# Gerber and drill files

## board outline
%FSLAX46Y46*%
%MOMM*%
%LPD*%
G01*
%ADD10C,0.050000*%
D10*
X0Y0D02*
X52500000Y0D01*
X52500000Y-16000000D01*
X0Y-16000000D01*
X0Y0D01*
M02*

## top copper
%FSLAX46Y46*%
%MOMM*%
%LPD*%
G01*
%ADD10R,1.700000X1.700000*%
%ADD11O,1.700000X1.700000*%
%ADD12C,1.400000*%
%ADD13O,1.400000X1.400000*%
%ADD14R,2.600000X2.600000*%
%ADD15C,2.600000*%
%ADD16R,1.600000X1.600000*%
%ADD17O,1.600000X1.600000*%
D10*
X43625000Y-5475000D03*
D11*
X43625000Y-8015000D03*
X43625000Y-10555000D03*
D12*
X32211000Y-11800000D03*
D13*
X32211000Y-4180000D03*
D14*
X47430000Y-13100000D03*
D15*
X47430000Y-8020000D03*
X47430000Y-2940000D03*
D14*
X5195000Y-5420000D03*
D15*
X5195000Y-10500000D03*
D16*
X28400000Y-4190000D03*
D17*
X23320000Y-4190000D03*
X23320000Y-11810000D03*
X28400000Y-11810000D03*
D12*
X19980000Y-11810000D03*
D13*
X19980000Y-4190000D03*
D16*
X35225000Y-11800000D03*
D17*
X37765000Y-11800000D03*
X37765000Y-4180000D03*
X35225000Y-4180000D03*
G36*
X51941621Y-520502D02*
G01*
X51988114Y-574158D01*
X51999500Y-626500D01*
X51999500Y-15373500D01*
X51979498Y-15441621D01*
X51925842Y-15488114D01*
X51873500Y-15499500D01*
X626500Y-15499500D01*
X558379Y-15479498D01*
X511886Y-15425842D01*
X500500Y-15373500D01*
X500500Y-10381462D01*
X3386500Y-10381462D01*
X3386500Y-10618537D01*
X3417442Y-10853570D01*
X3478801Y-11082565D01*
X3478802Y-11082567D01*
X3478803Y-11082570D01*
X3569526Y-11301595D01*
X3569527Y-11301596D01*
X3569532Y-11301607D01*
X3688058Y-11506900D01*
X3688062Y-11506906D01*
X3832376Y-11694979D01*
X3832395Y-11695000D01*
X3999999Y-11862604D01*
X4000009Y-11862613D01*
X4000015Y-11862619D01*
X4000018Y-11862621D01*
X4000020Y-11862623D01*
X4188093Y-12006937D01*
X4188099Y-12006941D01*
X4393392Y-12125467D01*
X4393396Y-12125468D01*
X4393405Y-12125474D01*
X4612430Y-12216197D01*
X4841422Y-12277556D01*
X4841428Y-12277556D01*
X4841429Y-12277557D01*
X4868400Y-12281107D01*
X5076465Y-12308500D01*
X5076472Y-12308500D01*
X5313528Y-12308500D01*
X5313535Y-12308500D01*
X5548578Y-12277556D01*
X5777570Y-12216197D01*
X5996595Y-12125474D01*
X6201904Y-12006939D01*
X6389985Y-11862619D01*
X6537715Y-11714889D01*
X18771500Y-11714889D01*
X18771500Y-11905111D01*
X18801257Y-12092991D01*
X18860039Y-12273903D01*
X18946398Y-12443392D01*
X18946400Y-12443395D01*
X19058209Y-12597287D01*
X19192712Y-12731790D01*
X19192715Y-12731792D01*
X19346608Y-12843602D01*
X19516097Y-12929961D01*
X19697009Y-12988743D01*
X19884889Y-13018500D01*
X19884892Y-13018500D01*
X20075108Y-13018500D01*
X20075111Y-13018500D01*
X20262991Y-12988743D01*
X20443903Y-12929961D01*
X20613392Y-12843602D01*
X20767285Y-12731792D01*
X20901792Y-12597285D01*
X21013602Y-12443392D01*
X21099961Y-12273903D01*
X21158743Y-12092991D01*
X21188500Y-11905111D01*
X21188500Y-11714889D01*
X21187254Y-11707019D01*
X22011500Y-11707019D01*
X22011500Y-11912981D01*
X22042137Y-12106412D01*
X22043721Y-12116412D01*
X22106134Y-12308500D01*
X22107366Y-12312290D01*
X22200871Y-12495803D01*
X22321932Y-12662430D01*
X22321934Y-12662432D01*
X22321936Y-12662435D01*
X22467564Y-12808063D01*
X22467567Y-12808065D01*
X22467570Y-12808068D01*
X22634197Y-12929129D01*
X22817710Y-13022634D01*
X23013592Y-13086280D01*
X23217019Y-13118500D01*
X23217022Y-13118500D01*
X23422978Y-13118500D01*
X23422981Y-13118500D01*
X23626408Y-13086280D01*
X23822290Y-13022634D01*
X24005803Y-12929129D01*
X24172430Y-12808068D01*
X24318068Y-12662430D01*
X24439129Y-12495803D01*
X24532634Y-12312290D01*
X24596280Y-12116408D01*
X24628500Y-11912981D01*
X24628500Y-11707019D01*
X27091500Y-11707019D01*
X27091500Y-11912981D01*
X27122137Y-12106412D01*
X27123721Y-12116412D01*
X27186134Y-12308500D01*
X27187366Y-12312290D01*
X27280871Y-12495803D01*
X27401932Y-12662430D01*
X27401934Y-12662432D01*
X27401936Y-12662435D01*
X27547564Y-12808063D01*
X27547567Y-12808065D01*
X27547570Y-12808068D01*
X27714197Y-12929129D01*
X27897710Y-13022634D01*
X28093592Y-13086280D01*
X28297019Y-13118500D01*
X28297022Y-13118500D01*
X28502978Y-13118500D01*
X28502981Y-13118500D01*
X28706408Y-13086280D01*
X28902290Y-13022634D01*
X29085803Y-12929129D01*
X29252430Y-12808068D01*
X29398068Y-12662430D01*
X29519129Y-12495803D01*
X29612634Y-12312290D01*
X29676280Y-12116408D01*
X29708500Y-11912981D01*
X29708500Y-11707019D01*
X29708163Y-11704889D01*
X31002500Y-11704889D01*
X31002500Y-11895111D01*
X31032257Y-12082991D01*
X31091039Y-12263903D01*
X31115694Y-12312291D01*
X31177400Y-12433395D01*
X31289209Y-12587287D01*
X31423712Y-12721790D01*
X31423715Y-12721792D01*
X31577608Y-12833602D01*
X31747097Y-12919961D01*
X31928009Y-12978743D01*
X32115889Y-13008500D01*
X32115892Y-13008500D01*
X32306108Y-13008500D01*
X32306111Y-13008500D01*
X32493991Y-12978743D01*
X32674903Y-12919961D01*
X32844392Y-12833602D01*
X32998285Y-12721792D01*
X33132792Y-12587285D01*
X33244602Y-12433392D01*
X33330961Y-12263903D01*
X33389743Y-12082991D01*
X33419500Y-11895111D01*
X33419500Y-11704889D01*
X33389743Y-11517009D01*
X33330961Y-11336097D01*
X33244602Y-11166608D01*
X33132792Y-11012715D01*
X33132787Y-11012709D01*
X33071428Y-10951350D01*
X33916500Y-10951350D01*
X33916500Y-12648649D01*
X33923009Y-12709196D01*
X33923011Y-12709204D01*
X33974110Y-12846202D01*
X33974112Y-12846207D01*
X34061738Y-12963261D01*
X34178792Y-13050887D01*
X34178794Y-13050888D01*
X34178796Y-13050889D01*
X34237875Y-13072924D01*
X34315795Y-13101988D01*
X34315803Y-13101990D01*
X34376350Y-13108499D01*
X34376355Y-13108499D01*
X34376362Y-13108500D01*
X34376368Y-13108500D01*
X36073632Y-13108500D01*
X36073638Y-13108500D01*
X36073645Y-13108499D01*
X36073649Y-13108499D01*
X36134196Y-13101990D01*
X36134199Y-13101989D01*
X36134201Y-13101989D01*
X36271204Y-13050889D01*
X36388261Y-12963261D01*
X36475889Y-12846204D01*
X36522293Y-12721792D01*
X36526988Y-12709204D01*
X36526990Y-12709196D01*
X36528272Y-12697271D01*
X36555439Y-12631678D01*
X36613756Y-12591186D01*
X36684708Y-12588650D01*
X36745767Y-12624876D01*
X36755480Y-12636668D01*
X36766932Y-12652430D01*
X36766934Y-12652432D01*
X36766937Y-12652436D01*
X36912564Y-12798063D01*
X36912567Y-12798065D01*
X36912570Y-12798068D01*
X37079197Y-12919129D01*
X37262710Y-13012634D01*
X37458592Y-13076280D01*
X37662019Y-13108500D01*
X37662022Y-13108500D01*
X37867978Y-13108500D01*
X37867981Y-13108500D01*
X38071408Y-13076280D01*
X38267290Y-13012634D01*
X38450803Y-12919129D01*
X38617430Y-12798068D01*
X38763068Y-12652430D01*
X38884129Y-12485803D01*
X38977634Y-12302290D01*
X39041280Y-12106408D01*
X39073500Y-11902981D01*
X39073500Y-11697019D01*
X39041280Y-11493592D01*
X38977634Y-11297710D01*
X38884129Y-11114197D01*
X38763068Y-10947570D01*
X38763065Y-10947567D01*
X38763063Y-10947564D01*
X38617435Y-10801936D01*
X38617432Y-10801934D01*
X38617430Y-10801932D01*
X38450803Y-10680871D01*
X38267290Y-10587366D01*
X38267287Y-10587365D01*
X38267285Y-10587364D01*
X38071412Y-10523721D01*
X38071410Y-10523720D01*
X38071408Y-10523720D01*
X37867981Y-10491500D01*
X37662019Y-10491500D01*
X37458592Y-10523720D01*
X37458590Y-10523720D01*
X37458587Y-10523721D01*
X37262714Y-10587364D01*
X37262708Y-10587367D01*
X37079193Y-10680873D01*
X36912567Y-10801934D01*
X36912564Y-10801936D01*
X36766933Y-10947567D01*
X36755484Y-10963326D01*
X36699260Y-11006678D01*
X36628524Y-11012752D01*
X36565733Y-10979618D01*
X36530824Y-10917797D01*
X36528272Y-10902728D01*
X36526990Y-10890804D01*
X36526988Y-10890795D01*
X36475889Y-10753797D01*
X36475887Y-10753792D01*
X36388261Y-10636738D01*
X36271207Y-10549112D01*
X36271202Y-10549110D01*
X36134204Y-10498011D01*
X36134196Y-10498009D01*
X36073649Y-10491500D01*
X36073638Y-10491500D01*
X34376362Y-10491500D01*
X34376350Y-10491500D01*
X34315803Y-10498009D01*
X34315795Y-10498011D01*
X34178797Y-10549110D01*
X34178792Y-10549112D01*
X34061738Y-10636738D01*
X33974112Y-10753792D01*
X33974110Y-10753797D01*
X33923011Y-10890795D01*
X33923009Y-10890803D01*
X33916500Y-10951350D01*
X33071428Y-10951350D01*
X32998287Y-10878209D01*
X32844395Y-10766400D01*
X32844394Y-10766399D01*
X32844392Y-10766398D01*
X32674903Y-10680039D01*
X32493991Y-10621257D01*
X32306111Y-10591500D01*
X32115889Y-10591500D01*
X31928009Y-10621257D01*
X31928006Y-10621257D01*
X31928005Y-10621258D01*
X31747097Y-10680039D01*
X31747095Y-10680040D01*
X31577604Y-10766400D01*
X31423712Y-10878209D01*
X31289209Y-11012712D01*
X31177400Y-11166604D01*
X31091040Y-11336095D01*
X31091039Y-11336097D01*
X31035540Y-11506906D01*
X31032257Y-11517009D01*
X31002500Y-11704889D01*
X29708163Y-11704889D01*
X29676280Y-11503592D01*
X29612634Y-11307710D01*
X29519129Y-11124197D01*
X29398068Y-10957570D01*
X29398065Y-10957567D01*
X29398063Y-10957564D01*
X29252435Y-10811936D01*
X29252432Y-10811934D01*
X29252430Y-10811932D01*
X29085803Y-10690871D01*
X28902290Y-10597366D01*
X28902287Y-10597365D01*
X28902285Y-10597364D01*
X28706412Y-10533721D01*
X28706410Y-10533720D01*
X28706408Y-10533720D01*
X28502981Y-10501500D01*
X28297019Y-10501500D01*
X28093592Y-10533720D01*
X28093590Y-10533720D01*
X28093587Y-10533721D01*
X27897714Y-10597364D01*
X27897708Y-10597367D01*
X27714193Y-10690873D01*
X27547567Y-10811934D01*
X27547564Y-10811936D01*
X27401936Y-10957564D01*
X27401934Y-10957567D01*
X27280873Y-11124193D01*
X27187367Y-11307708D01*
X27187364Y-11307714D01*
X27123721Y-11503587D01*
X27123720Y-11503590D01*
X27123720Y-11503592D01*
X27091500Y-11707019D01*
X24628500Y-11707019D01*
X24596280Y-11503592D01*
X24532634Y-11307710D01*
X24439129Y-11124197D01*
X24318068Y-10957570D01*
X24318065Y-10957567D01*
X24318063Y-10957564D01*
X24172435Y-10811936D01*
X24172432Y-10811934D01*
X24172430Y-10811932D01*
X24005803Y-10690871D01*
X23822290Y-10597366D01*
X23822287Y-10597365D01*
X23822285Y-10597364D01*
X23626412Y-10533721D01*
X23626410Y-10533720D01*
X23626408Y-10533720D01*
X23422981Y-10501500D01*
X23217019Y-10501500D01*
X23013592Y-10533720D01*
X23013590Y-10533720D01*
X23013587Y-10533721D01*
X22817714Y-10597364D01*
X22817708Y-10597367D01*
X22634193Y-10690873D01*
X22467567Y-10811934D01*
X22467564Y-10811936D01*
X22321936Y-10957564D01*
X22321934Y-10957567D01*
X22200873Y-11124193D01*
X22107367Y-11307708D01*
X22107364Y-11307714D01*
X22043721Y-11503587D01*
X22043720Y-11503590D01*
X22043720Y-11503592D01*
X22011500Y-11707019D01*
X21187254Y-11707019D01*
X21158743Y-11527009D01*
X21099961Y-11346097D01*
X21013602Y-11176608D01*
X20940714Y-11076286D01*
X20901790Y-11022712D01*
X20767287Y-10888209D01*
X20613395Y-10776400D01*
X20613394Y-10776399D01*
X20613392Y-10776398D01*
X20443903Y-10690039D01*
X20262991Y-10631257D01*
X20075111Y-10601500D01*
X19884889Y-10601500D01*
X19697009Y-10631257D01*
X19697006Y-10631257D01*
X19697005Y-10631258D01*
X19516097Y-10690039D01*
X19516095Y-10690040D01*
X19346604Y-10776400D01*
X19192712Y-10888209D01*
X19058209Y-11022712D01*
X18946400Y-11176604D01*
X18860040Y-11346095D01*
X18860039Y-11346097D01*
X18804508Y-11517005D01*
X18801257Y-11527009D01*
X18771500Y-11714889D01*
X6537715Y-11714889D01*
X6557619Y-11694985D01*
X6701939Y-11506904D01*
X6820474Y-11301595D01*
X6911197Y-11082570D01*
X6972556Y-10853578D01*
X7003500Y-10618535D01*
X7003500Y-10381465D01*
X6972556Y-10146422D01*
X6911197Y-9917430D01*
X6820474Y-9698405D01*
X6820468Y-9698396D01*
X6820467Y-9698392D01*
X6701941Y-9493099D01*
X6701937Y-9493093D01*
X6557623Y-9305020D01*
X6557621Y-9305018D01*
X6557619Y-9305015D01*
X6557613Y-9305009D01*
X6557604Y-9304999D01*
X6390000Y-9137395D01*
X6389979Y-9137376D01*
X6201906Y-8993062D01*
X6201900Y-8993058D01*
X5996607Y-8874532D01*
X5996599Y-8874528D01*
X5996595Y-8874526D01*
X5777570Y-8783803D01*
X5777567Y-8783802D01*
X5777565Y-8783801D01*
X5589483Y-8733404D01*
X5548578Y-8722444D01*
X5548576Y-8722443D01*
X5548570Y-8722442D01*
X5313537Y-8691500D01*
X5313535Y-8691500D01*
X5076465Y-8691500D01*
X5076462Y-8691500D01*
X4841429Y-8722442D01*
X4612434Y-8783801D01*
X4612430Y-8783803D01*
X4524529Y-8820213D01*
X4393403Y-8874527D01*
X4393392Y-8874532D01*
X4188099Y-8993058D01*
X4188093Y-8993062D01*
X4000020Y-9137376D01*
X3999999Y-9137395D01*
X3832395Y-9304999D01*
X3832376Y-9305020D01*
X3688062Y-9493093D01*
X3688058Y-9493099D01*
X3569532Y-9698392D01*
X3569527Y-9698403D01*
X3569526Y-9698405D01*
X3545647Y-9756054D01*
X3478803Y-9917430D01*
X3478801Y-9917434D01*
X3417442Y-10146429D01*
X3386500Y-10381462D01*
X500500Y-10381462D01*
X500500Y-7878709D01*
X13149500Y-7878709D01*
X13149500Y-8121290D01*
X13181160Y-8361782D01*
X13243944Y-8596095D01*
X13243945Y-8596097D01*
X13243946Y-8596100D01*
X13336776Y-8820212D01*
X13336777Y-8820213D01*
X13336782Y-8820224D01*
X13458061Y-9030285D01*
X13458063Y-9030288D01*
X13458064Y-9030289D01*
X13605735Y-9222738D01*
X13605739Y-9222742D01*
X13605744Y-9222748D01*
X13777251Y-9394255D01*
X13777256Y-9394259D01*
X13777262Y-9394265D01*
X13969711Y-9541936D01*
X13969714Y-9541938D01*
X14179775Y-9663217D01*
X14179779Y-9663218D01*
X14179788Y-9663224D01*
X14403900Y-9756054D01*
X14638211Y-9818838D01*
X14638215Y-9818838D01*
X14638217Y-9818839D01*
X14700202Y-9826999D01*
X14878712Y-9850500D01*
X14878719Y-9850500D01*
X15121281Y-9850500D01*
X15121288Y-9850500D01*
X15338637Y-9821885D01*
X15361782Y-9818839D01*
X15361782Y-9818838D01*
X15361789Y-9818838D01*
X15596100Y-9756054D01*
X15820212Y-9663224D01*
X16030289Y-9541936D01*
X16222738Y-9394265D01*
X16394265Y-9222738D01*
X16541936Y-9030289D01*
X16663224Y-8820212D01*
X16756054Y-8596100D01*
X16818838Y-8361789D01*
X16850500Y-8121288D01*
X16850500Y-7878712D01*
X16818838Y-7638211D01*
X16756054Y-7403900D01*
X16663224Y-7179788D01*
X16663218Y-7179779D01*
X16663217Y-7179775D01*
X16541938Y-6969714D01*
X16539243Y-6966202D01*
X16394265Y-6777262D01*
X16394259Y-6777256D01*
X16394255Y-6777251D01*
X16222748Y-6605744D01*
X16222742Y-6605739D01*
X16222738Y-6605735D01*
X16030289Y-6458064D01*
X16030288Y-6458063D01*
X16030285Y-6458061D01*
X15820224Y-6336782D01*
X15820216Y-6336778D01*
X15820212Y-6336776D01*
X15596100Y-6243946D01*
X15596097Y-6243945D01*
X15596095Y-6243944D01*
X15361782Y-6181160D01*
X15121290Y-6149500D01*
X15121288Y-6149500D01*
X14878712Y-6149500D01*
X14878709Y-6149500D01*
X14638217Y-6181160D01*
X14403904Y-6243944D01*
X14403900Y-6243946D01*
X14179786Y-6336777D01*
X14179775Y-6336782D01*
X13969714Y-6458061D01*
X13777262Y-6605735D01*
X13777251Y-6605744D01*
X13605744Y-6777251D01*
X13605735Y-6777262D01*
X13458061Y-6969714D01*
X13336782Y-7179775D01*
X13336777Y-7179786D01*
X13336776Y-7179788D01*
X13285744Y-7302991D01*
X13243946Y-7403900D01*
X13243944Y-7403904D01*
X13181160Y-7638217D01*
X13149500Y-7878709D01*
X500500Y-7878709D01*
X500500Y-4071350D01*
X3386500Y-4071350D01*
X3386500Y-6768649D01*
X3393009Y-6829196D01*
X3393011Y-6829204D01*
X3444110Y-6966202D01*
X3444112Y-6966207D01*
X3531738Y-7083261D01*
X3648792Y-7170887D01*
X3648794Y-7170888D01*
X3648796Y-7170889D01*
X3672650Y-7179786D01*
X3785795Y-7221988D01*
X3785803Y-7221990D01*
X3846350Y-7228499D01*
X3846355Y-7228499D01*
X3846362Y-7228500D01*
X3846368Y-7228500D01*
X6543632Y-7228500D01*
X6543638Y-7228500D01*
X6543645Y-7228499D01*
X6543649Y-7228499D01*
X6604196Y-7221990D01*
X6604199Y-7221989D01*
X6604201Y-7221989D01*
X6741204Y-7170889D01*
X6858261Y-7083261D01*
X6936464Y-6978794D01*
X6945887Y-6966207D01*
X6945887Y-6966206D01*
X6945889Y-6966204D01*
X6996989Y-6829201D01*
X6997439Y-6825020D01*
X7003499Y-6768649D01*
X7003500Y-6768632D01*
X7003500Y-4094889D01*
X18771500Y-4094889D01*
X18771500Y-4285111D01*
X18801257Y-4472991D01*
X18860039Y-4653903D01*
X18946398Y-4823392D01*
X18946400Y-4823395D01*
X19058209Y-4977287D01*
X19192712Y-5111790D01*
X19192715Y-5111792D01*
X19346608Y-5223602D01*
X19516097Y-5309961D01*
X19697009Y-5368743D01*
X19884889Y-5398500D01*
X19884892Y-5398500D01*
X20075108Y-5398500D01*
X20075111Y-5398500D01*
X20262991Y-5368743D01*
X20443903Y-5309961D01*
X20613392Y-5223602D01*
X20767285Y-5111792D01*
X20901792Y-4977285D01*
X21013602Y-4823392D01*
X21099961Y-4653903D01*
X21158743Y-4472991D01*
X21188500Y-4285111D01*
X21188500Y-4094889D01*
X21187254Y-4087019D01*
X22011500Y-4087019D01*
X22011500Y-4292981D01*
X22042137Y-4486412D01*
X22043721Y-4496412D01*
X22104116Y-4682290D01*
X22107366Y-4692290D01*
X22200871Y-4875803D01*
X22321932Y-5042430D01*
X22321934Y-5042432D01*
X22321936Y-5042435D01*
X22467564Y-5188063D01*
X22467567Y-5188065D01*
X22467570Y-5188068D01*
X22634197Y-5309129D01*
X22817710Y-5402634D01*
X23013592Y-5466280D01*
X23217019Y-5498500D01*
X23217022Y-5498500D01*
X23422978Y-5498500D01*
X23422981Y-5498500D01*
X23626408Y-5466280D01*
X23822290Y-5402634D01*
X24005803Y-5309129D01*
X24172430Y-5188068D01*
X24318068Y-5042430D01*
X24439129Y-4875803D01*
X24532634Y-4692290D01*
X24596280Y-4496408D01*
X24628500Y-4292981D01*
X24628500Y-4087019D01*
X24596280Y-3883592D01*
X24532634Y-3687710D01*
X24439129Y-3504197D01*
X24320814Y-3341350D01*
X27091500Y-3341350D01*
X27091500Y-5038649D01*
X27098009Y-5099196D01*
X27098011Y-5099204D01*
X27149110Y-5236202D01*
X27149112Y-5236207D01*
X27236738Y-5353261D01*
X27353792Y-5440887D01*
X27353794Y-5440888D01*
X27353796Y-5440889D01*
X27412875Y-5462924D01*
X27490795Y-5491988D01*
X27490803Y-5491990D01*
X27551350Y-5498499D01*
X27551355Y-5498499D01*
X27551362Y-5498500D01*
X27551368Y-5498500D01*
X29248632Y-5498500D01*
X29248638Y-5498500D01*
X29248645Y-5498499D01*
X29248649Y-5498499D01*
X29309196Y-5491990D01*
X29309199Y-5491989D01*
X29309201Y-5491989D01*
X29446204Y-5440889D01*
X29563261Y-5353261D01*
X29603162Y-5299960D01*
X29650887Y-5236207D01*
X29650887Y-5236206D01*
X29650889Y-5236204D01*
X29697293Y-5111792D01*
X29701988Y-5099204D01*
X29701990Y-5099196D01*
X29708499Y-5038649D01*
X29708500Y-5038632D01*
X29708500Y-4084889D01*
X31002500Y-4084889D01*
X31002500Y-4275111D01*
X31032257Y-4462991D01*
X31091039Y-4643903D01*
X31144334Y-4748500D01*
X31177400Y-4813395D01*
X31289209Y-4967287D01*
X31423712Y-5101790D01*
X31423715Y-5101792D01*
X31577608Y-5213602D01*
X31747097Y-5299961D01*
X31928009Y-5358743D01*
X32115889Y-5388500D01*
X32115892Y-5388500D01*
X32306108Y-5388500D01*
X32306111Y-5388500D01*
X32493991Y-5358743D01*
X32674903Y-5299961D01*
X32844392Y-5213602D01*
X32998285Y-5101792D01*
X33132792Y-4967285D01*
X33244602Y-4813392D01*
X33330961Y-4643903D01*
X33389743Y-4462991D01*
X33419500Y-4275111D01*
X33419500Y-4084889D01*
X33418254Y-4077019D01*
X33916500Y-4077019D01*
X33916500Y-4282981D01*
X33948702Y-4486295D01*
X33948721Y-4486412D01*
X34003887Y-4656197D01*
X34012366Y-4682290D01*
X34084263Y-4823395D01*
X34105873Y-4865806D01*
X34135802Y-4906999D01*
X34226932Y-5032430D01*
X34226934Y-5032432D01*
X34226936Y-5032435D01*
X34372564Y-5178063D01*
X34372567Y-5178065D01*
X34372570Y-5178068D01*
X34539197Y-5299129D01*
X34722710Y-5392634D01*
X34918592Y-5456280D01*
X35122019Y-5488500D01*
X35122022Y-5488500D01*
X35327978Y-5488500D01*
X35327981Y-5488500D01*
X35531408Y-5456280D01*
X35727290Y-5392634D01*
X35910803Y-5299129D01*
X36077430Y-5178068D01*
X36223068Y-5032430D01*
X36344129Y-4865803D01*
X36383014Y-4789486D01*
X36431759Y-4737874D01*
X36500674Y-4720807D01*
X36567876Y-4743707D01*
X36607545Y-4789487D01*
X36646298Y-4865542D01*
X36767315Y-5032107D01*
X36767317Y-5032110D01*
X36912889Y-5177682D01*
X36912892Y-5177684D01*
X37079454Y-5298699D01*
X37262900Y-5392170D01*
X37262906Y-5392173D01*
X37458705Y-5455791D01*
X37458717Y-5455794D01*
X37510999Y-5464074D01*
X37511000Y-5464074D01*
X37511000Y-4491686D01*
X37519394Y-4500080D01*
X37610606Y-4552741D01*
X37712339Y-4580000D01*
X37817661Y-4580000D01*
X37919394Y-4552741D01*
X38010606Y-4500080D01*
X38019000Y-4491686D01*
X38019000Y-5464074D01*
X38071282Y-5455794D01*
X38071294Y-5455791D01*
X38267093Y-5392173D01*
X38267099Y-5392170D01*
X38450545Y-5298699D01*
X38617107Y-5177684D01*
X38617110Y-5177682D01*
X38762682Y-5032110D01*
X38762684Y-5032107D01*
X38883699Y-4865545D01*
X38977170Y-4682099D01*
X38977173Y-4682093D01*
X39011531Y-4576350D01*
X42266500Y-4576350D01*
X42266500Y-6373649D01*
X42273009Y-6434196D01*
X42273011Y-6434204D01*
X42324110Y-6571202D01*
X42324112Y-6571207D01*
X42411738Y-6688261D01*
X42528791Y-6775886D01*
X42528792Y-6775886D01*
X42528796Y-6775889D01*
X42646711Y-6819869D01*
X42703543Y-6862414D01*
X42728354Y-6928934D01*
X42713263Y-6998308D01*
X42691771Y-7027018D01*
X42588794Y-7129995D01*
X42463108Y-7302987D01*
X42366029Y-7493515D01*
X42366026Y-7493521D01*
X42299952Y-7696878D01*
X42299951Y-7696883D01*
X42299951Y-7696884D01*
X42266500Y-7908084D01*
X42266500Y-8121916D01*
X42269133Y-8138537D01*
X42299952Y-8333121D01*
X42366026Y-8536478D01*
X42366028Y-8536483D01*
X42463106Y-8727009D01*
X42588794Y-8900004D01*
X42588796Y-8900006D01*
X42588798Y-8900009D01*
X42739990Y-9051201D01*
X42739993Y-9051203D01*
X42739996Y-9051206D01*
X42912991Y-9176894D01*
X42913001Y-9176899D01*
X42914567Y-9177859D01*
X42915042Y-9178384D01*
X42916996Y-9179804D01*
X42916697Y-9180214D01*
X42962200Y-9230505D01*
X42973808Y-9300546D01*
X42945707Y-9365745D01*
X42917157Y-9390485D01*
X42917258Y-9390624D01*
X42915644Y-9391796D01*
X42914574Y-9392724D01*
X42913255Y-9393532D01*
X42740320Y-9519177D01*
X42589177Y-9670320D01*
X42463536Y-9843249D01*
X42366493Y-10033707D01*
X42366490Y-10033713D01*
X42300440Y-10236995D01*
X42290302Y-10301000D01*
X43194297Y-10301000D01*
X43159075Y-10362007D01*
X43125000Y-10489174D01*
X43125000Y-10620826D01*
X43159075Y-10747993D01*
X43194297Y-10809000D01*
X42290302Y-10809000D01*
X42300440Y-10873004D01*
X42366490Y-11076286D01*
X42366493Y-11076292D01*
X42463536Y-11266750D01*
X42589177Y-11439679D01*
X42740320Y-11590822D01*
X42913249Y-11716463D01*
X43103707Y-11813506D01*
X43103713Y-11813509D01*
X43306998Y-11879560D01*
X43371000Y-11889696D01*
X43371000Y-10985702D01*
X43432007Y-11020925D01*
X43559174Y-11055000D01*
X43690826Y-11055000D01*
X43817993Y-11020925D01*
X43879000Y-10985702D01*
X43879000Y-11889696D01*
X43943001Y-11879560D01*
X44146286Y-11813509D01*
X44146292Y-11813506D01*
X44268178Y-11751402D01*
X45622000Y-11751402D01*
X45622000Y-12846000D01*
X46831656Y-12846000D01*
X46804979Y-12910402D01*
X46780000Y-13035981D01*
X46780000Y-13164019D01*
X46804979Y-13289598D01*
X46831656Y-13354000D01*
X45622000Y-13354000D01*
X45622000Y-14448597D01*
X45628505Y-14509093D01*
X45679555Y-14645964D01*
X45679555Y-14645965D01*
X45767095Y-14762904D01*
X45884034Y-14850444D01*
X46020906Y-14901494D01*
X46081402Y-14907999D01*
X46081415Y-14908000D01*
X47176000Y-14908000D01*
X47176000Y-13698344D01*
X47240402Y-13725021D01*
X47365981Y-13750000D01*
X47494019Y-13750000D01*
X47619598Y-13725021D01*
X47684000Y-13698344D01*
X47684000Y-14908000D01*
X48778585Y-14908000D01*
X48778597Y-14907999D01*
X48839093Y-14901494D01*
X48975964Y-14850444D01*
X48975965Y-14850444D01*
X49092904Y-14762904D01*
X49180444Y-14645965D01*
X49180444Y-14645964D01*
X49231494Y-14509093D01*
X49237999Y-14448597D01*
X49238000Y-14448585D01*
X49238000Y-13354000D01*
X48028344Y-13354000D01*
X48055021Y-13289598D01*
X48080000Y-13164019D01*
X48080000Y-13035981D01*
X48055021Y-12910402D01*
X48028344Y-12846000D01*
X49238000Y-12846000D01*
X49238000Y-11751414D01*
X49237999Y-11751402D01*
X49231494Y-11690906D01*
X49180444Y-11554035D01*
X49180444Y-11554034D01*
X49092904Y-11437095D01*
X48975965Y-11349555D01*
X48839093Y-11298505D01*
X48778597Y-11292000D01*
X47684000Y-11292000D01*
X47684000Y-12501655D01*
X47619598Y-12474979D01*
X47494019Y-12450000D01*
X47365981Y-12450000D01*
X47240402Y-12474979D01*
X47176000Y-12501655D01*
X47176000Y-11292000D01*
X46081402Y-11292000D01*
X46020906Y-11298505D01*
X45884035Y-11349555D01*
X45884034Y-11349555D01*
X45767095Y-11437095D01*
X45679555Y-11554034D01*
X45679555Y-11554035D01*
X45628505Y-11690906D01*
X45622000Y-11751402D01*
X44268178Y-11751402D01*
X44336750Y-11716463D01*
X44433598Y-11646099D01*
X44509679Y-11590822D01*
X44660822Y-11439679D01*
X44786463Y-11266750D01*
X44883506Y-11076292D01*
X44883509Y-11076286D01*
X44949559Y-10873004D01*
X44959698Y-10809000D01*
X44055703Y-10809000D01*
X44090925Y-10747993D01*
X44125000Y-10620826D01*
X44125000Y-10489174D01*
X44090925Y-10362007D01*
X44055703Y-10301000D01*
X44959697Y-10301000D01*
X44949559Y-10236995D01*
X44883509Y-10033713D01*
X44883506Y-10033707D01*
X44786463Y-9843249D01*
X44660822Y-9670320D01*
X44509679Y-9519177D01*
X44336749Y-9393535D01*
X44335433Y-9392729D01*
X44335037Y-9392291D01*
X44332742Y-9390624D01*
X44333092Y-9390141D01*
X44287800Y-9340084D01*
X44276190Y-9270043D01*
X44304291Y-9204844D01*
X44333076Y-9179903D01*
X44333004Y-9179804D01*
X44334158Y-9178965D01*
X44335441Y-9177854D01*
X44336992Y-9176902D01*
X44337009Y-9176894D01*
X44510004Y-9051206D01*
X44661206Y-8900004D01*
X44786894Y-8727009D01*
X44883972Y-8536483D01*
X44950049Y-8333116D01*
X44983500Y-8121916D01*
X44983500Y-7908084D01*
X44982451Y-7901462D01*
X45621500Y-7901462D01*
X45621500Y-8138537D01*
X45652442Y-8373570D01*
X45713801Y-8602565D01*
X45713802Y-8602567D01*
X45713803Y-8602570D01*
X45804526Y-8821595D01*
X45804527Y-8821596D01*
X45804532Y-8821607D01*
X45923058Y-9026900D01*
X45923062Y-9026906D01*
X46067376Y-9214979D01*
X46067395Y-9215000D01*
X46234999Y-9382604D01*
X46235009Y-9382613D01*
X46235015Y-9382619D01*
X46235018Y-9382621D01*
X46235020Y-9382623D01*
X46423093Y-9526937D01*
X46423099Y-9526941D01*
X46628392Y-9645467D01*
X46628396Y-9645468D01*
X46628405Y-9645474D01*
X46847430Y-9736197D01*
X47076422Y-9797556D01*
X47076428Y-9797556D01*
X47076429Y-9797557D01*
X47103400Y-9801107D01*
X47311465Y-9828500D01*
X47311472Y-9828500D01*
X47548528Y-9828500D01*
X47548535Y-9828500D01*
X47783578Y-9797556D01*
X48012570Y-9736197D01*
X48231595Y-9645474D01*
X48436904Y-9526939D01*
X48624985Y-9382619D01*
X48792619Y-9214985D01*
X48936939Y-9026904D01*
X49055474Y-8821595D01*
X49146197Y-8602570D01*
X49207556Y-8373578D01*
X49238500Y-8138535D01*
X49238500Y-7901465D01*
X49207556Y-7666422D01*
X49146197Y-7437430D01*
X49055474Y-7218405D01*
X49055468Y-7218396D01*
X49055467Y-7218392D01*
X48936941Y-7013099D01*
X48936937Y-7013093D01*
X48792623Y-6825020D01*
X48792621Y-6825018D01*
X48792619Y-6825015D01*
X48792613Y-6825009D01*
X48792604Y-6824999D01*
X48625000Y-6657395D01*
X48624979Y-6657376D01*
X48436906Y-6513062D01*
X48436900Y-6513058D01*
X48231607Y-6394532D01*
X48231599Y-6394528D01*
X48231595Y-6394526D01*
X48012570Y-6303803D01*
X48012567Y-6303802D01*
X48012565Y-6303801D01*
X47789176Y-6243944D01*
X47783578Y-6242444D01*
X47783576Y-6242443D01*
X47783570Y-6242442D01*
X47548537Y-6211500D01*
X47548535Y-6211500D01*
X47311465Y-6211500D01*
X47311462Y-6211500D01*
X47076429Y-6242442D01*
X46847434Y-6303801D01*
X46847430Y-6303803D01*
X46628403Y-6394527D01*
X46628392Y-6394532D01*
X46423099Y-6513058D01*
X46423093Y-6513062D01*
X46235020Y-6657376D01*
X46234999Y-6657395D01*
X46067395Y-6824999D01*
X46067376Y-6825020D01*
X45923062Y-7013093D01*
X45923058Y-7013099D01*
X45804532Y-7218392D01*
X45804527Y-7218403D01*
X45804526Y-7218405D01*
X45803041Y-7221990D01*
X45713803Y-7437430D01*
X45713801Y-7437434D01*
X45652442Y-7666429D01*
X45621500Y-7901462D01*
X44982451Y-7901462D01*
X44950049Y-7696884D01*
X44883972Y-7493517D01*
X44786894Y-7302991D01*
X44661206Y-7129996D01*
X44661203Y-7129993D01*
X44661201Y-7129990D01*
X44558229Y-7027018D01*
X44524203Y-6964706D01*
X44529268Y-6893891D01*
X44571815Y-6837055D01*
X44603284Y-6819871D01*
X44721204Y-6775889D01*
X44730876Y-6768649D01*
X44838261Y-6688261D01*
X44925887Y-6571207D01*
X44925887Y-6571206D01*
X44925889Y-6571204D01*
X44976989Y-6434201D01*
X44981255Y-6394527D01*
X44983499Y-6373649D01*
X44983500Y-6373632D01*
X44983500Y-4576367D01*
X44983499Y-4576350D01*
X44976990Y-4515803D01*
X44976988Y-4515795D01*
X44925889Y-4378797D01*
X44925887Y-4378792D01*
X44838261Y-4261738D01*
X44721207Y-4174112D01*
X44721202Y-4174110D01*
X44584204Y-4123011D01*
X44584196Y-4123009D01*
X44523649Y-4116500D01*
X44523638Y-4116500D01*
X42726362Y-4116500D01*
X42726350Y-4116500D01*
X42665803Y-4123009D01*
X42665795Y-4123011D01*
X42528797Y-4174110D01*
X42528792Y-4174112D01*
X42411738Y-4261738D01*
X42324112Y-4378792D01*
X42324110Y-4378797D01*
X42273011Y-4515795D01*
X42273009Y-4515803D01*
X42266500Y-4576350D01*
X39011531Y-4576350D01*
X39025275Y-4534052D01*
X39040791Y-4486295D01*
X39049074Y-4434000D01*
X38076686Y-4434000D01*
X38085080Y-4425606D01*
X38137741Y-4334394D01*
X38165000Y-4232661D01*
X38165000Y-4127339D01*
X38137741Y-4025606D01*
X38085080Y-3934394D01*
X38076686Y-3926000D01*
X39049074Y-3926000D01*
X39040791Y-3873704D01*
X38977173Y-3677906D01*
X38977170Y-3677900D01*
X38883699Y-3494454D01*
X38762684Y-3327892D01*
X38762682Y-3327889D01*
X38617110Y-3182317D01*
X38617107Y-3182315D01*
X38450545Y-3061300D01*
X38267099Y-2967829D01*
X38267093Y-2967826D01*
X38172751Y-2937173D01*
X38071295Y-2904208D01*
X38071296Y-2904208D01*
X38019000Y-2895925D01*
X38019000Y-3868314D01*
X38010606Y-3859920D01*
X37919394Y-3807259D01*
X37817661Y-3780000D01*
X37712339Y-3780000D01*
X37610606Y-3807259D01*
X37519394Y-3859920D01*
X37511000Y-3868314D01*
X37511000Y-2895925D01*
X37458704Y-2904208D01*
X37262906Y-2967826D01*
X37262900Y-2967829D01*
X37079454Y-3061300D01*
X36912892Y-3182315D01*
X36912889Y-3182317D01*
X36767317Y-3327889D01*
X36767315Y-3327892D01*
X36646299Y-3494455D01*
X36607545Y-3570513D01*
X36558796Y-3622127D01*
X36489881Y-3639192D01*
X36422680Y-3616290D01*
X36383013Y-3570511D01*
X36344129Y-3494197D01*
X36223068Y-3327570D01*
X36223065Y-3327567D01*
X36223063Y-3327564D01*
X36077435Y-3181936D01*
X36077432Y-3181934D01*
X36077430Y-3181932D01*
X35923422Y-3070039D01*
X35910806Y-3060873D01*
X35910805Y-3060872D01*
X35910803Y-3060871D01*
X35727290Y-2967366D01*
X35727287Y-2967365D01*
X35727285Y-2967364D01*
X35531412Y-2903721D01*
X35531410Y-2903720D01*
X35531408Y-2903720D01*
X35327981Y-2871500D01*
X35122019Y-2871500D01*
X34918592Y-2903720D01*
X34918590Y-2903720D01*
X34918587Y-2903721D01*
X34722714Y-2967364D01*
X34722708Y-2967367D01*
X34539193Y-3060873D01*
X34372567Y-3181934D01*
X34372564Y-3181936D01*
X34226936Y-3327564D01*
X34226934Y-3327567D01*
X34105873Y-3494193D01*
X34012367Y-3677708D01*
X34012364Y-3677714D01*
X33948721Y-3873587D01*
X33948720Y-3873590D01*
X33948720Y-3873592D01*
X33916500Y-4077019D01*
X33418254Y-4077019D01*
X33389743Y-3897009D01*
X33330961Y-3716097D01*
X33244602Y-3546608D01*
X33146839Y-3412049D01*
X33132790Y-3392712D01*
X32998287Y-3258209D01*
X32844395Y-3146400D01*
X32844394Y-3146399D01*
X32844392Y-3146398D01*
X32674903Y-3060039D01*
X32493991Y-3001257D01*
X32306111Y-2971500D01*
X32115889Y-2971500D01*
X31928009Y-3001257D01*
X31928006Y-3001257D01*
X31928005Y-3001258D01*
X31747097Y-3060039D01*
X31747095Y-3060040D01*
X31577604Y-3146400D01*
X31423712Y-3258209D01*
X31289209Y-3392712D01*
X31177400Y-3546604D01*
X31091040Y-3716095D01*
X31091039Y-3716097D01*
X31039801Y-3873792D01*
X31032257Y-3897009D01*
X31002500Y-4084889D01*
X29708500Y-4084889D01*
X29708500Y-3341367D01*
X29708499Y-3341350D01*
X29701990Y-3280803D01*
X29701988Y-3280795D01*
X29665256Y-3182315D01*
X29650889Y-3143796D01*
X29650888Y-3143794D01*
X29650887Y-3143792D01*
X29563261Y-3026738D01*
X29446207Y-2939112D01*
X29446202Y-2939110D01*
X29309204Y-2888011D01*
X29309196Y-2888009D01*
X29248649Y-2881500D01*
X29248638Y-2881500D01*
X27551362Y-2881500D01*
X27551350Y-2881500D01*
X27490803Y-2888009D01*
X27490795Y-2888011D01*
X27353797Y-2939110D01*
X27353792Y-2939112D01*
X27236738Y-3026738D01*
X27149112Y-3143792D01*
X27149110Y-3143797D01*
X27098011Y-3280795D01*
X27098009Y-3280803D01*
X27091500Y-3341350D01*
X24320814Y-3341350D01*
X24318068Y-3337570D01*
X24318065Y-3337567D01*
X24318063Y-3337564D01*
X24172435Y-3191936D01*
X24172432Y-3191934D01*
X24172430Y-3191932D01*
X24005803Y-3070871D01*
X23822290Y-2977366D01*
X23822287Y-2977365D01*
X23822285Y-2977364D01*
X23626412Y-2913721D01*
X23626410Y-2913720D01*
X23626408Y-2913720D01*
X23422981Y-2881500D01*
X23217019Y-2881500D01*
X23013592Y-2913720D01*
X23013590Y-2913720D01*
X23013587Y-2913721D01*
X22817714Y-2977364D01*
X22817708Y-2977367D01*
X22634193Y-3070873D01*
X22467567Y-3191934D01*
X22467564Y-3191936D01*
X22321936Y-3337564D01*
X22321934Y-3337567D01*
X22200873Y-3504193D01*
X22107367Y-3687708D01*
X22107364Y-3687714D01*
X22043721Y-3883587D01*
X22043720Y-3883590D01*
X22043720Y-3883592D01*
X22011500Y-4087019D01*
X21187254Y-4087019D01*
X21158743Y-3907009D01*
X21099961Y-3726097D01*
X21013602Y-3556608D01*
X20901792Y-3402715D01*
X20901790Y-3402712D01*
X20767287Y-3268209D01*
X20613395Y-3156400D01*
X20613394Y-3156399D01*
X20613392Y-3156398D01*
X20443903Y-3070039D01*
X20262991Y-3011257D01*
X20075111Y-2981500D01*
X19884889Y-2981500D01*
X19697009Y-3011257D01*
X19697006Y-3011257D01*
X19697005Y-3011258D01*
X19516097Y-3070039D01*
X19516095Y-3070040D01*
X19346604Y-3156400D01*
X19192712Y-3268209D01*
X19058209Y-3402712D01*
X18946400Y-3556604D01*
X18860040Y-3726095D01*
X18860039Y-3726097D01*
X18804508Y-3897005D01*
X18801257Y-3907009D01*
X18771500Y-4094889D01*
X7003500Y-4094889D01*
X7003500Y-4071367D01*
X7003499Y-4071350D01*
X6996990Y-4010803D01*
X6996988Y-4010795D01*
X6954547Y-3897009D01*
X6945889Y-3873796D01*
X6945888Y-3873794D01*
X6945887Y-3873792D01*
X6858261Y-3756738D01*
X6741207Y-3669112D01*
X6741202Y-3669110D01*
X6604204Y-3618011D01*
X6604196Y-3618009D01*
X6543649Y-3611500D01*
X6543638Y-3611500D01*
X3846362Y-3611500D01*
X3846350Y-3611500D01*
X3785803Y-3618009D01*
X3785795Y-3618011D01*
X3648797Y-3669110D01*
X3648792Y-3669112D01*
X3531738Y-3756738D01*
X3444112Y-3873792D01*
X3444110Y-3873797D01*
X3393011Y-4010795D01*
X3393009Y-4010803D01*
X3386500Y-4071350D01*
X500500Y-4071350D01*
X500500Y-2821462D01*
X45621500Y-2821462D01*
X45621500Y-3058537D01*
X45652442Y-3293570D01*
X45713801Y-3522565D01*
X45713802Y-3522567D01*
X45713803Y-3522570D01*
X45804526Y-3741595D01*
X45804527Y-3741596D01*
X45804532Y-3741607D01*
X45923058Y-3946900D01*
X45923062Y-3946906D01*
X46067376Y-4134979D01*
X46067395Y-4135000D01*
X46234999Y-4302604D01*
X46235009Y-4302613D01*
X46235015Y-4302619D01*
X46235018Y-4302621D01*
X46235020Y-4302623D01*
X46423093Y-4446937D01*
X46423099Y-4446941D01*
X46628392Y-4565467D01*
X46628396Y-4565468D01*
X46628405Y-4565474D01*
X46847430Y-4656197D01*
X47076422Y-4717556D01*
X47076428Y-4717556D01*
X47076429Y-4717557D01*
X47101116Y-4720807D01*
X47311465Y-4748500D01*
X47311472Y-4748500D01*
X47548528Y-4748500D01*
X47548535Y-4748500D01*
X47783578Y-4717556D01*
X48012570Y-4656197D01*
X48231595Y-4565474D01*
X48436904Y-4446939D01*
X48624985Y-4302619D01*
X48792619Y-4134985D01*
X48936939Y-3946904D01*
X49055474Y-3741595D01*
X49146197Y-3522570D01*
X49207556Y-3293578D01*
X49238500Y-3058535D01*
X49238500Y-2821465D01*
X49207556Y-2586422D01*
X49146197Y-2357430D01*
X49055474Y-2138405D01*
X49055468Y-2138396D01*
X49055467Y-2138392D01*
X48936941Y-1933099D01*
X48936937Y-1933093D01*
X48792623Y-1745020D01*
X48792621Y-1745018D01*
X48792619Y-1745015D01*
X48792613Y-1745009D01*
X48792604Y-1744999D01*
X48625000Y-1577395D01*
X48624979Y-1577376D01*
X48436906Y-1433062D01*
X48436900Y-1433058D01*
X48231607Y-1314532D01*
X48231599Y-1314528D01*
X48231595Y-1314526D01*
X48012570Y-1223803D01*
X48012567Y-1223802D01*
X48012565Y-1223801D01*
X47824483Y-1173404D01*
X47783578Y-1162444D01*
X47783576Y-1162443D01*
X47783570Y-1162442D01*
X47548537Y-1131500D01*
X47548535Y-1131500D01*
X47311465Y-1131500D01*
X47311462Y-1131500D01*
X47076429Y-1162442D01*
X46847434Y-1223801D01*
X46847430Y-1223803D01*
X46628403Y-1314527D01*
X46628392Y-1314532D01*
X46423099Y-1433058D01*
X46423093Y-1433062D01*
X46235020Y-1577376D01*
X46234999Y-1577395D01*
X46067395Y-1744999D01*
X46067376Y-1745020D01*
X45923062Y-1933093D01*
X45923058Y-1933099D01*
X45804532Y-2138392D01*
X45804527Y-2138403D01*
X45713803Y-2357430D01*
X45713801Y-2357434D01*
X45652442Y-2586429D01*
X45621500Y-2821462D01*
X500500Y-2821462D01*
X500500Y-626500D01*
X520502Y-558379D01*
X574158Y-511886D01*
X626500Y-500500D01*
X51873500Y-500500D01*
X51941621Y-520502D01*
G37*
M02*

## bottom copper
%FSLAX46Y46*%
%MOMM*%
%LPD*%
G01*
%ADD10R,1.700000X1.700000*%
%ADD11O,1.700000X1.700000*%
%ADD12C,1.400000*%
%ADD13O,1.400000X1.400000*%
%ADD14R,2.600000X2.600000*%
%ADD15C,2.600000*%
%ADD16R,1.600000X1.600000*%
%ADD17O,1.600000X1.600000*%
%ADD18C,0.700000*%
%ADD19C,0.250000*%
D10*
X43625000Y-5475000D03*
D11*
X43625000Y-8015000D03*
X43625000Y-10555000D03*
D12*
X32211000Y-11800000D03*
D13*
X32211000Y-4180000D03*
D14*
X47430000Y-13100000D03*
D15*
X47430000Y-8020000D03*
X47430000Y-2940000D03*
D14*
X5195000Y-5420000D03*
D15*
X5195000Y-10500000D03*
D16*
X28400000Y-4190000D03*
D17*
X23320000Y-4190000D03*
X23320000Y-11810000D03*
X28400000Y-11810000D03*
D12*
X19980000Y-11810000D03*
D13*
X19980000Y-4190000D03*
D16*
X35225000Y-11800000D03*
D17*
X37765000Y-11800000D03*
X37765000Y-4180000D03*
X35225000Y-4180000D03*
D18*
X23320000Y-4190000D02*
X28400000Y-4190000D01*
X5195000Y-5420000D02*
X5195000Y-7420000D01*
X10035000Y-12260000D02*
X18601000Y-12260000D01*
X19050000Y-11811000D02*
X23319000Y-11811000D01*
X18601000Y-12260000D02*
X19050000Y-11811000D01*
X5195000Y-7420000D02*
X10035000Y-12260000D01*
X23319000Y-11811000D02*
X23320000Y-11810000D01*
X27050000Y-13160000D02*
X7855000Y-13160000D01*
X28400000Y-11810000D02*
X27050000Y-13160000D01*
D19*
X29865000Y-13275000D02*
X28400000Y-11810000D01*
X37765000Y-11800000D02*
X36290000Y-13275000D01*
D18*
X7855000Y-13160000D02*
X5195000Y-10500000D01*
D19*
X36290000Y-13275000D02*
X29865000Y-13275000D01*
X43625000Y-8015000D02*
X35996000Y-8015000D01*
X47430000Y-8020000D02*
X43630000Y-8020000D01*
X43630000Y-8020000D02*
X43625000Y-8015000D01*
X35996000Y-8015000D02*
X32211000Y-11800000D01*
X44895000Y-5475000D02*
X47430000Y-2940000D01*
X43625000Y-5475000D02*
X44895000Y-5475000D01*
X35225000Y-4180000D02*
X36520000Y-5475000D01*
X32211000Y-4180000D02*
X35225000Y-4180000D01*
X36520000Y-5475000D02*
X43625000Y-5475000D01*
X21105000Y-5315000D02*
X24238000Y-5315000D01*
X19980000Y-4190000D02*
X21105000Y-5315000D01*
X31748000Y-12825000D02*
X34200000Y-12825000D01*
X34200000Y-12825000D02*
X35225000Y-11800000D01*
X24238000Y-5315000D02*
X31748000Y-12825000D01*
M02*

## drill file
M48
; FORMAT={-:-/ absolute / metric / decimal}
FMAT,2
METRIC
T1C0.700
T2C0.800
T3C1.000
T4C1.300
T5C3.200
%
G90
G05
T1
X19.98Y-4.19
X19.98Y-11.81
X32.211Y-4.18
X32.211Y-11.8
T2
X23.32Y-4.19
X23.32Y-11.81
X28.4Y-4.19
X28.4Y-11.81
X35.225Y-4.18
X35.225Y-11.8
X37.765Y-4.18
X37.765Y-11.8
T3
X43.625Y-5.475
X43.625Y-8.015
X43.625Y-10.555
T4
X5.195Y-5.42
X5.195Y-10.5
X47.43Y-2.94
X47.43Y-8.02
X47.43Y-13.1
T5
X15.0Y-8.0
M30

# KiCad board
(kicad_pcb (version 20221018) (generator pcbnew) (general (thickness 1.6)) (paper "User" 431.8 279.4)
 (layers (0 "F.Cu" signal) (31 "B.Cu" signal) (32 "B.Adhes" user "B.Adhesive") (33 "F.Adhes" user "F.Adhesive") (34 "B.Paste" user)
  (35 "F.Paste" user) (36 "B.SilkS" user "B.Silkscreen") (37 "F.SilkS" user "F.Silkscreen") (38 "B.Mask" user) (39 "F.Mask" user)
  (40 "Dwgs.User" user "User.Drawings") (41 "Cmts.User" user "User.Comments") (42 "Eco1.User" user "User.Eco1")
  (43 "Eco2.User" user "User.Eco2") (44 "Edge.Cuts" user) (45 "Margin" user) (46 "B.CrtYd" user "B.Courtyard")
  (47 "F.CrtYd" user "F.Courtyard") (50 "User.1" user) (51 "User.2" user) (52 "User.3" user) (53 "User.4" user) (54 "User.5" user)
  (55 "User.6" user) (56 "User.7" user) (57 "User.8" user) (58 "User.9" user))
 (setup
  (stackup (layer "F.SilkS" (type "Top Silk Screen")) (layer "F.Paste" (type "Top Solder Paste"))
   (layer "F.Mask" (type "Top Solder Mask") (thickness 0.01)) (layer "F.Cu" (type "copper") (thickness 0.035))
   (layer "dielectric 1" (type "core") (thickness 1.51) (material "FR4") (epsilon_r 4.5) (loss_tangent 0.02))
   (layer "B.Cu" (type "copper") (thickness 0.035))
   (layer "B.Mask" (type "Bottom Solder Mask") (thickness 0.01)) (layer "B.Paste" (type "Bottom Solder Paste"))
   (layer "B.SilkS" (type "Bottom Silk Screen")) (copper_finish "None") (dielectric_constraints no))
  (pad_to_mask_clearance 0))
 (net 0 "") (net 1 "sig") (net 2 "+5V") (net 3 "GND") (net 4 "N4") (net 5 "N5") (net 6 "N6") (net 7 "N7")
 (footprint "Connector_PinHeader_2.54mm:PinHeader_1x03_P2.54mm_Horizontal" (layer "F.Cu") (at 43.625 5.475)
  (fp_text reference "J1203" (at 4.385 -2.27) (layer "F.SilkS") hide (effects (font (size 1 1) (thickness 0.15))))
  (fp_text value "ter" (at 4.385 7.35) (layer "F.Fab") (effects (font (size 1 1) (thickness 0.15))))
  (pad "1" thru_hole rect (at 0 0) (size 1.7 1.7) (drill 1) (layers "*.Cu" "*.Mask") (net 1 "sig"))
  (pad "2" thru_hole oval (at 0 2.54) (size 1.7 1.7) (drill 1) (layers "*.Cu" "*.Mask") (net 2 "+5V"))
  (pad "3" thru_hole oval (at 0 5.08) (size 1.7 1.7) (drill 1) (layers "*.Cu" "*.Mask") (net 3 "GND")))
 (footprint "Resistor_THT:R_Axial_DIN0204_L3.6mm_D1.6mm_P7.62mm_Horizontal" (layer "F.Cu") (at 32.211 11.8 90)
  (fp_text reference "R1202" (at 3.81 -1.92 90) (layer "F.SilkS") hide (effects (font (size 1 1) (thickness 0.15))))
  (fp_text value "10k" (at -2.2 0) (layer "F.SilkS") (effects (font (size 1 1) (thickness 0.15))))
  (pad "1" thru_hole circle (at 0 0 90) (size 1.4 1.4) (drill 0.7) (layers "*.Cu" "*.Mask") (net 2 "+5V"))
  (pad "2" thru_hole oval (at 7.62 0 90) (size 1.4 1.4) (drill 0.7) (layers "*.Cu" "*.Mask") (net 1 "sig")))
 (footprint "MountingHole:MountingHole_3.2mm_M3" (layer "F.Cu") (at 15 8)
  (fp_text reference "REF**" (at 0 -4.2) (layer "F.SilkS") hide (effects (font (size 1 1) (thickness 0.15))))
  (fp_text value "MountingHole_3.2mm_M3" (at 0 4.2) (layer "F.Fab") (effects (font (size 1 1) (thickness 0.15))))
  (pad "" np_thru_hole circle (at 0 0) (size 3.2 3.2) (drill 3.2) (layers "*.Cu" "*.Mask")))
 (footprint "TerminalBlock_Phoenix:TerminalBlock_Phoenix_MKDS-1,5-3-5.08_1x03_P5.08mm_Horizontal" (layer "F.Cu") (at 47.43 13.1 90)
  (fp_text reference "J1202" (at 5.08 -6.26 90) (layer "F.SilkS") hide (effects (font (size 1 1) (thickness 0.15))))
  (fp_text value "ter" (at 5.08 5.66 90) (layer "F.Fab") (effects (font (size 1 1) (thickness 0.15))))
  (pad "1" thru_hole rect (at 0 0 90) (size 2.6 2.6) (drill 1.3) (layers "*.Cu" "*.Mask") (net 3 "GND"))
  (pad "2" thru_hole circle (at 5.08 0 90) (size 2.6 2.6) (drill 1.3) (layers "*.Cu" "*.Mask") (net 2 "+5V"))
  (pad "3" thru_hole circle (at 10.16 0 90) (size 2.6 2.6) (drill 1.3) (layers "*.Cu" "*.Mask") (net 1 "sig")))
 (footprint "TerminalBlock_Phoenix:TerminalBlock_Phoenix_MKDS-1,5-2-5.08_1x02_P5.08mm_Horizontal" (layer "F.Cu") (at 5.195 5.42 -90)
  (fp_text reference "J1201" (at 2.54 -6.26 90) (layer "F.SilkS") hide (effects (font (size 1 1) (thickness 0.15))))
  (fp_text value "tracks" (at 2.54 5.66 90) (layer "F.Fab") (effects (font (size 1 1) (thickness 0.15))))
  (pad "1" thru_hole rect (at 0 0 270) (size 2.6 2.6) (drill 1.3) (layers "*.Cu" "*.Mask") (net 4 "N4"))
  (pad "2" thru_hole circle (at 5.08 0 270) (size 2.6 2.6) (drill 1.3) (layers "*.Cu" "*.Mask") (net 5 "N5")))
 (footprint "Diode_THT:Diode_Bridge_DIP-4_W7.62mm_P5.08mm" (layer "F.Cu") (at 28.4 4.19 -90)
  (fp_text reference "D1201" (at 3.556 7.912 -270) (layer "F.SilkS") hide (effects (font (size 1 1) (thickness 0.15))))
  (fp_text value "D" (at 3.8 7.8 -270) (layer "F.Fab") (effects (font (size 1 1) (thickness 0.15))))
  (pad "1" thru_hole rect (at 0 0 270) (size 1.6 1.6) (drill 0.8) (layers "*.Cu" "*.Mask") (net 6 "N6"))
  (pad "2" thru_hole oval (at 0 5.08 270) (size 1.6 1.6) (drill 0.8) (layers "*.Cu" "*.Mask") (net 6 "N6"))
  (pad "3" thru_hole oval (at 7.62 5.08 270) (size 1.6 1.6) (drill 0.8) (layers "*.Cu" "*.Mask") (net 4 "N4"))
  (pad "4" thru_hole oval (at 7.62 0 270) (size 1.6 1.6) (drill 0.8) (layers "*.Cu" "*.Mask") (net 5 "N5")))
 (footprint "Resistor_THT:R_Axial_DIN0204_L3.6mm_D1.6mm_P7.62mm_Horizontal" (layer "F.Cu") (at 19.98 11.81 90)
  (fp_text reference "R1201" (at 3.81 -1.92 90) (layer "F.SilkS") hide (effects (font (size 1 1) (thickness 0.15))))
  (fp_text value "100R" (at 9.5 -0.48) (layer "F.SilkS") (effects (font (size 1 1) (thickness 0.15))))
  (pad "1" thru_hole circle (at 0 0 90) (size 1.4 1.4) (drill 0.7) (layers "*.Cu" "*.Mask") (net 4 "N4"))
  (pad "2" thru_hole oval (at 7.62 0 90) (size 1.4 1.4) (drill 0.7) (layers "*.Cu" "*.Mask") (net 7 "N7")))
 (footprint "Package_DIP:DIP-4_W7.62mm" (layer "F.Cu") (at 35.225 11.8 90)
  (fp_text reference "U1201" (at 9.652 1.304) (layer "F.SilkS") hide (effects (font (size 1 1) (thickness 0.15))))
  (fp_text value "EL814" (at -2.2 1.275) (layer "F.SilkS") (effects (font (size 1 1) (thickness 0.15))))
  (pad "1" thru_hole rect (at 0 0 90) (size 1.6 1.6) (drill 0.8) (layers "*.Cu" "*.Mask") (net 7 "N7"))
  (pad "2" thru_hole oval (at 0 2.54 90) (size 1.6 1.6) (drill 0.8) (layers "*.Cu" "*.Mask") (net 5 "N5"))
  (pad "3" thru_hole oval (at 7.62 2.54 90) (size 1.6 1.6) (drill 0.8) (layers "*.Cu" "*.Mask") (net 3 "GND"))
  (pad "4" thru_hole oval (at 7.62 0 90) (size 1.6 1.6) (drill 0.8) (layers "*.Cu" "*.Mask") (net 1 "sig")))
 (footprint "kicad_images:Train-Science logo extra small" (layer "B.Cu") (at 28 8 -90)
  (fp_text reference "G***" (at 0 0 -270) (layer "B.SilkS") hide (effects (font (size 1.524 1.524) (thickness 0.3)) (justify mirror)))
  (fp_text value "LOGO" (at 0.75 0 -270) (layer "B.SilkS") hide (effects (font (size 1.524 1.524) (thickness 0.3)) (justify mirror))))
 (gr_rect (start 0 0) (end 52.5 16) (stroke (width 0.05) (type default)) (fill none) (layer "Edge.Cuts"))
 (segment (start 23.32 4.19) (end 28.4 4.19) (width 0.7) (layer "B.Cu") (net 6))
 (segment (start 5.195 5.42) (end 5.195 7.42) (width 0.7) (layer "B.Cu") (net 4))
 (segment (start 10.035 12.26) (end 18.601 12.26) (width 0.7) (layer "B.Cu") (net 4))
 (segment (start 19.05 11.811) (end 23.319 11.811) (width 0.7) (layer "B.Cu") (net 4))
 (segment (start 18.601 12.26) (end 19.05 11.811) (width 0.7) (layer "B.Cu") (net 4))
 (segment (start 5.195 7.42) (end 10.035 12.26) (width 0.7) (layer "B.Cu") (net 4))
 (segment (start 23.319 11.811) (end 23.32 11.81) (width 0.7) (layer "B.Cu") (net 4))
 (segment (start 27.05 13.16) (end 7.855 13.16) (width 0.7) (layer "B.Cu") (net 5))
 (segment (start 28.4 11.81) (end 27.05 13.16) (width 0.7) (layer "B.Cu") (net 5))
 (segment (start 29.865 13.275) (end 28.4 11.81) (width 0.25) (layer "B.Cu") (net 5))
 (segment (start 37.765 11.8) (end 36.29 13.275) (width 0.25) (layer "B.Cu") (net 5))
 (segment (start 7.855 13.16) (end 5.195 10.5) (width 0.7) (layer "B.Cu") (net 5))
 (segment (start 36.29 13.275) (end 29.865 13.275) (width 0.25) (layer "B.Cu") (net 5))
 (segment (start 43.625 8.015) (end 35.996 8.015) (width 0.25) (layer "B.Cu") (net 2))
 (segment (start 47.43 8.02) (end 43.63 8.02) (width 0.25) (layer "B.Cu") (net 2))
 (segment (start 43.63 8.02) (end 43.625 8.015) (width 0.25) (layer "B.Cu") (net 2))
 (segment (start 35.996 8.015) (end 32.211 11.8) (width 0.25) (layer "B.Cu") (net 2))
 (segment (start 44.895 5.475) (end 47.43 2.94) (width 0.25) (layer "B.Cu") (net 1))
 (segment (start 43.625 5.475) (end 44.895 5.475) (width 0.25) (layer "B.Cu") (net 1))
 (segment (start 35.225 4.18) (end 36.52 5.475) (width 0.25) (layer "B.Cu") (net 1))
 (segment (start 32.211 4.18) (end 35.225 4.18) (width 0.25) (layer "B.Cu") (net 1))
 (segment (start 36.52 5.475) (end 43.625 5.475) (width 0.25) (layer "B.Cu") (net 1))
 (segment (start 21.105 5.315) (end 24.238 5.315) (width 0.25) (layer "B.Cu") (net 7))
 (segment (start 19.98 4.19) (end 21.105 5.315) (width 0.25) (layer "B.Cu") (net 7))
 (segment (start 31.748 12.825) (end 34.2 12.825) (width 0.25) (layer "B.Cu") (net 7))
 (segment (start 34.2 12.825) (end 35.225 11.8) (width 0.25) (layer "B.Cu") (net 7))
 (segment (start 24.238 5.315) (end 31.748 12.825) (width 0.25) (layer "B.Cu") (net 7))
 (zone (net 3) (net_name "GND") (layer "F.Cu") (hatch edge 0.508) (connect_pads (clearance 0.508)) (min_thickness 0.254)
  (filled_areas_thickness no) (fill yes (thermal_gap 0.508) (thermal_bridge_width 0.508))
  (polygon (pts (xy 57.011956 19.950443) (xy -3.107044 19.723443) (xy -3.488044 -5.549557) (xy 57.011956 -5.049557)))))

